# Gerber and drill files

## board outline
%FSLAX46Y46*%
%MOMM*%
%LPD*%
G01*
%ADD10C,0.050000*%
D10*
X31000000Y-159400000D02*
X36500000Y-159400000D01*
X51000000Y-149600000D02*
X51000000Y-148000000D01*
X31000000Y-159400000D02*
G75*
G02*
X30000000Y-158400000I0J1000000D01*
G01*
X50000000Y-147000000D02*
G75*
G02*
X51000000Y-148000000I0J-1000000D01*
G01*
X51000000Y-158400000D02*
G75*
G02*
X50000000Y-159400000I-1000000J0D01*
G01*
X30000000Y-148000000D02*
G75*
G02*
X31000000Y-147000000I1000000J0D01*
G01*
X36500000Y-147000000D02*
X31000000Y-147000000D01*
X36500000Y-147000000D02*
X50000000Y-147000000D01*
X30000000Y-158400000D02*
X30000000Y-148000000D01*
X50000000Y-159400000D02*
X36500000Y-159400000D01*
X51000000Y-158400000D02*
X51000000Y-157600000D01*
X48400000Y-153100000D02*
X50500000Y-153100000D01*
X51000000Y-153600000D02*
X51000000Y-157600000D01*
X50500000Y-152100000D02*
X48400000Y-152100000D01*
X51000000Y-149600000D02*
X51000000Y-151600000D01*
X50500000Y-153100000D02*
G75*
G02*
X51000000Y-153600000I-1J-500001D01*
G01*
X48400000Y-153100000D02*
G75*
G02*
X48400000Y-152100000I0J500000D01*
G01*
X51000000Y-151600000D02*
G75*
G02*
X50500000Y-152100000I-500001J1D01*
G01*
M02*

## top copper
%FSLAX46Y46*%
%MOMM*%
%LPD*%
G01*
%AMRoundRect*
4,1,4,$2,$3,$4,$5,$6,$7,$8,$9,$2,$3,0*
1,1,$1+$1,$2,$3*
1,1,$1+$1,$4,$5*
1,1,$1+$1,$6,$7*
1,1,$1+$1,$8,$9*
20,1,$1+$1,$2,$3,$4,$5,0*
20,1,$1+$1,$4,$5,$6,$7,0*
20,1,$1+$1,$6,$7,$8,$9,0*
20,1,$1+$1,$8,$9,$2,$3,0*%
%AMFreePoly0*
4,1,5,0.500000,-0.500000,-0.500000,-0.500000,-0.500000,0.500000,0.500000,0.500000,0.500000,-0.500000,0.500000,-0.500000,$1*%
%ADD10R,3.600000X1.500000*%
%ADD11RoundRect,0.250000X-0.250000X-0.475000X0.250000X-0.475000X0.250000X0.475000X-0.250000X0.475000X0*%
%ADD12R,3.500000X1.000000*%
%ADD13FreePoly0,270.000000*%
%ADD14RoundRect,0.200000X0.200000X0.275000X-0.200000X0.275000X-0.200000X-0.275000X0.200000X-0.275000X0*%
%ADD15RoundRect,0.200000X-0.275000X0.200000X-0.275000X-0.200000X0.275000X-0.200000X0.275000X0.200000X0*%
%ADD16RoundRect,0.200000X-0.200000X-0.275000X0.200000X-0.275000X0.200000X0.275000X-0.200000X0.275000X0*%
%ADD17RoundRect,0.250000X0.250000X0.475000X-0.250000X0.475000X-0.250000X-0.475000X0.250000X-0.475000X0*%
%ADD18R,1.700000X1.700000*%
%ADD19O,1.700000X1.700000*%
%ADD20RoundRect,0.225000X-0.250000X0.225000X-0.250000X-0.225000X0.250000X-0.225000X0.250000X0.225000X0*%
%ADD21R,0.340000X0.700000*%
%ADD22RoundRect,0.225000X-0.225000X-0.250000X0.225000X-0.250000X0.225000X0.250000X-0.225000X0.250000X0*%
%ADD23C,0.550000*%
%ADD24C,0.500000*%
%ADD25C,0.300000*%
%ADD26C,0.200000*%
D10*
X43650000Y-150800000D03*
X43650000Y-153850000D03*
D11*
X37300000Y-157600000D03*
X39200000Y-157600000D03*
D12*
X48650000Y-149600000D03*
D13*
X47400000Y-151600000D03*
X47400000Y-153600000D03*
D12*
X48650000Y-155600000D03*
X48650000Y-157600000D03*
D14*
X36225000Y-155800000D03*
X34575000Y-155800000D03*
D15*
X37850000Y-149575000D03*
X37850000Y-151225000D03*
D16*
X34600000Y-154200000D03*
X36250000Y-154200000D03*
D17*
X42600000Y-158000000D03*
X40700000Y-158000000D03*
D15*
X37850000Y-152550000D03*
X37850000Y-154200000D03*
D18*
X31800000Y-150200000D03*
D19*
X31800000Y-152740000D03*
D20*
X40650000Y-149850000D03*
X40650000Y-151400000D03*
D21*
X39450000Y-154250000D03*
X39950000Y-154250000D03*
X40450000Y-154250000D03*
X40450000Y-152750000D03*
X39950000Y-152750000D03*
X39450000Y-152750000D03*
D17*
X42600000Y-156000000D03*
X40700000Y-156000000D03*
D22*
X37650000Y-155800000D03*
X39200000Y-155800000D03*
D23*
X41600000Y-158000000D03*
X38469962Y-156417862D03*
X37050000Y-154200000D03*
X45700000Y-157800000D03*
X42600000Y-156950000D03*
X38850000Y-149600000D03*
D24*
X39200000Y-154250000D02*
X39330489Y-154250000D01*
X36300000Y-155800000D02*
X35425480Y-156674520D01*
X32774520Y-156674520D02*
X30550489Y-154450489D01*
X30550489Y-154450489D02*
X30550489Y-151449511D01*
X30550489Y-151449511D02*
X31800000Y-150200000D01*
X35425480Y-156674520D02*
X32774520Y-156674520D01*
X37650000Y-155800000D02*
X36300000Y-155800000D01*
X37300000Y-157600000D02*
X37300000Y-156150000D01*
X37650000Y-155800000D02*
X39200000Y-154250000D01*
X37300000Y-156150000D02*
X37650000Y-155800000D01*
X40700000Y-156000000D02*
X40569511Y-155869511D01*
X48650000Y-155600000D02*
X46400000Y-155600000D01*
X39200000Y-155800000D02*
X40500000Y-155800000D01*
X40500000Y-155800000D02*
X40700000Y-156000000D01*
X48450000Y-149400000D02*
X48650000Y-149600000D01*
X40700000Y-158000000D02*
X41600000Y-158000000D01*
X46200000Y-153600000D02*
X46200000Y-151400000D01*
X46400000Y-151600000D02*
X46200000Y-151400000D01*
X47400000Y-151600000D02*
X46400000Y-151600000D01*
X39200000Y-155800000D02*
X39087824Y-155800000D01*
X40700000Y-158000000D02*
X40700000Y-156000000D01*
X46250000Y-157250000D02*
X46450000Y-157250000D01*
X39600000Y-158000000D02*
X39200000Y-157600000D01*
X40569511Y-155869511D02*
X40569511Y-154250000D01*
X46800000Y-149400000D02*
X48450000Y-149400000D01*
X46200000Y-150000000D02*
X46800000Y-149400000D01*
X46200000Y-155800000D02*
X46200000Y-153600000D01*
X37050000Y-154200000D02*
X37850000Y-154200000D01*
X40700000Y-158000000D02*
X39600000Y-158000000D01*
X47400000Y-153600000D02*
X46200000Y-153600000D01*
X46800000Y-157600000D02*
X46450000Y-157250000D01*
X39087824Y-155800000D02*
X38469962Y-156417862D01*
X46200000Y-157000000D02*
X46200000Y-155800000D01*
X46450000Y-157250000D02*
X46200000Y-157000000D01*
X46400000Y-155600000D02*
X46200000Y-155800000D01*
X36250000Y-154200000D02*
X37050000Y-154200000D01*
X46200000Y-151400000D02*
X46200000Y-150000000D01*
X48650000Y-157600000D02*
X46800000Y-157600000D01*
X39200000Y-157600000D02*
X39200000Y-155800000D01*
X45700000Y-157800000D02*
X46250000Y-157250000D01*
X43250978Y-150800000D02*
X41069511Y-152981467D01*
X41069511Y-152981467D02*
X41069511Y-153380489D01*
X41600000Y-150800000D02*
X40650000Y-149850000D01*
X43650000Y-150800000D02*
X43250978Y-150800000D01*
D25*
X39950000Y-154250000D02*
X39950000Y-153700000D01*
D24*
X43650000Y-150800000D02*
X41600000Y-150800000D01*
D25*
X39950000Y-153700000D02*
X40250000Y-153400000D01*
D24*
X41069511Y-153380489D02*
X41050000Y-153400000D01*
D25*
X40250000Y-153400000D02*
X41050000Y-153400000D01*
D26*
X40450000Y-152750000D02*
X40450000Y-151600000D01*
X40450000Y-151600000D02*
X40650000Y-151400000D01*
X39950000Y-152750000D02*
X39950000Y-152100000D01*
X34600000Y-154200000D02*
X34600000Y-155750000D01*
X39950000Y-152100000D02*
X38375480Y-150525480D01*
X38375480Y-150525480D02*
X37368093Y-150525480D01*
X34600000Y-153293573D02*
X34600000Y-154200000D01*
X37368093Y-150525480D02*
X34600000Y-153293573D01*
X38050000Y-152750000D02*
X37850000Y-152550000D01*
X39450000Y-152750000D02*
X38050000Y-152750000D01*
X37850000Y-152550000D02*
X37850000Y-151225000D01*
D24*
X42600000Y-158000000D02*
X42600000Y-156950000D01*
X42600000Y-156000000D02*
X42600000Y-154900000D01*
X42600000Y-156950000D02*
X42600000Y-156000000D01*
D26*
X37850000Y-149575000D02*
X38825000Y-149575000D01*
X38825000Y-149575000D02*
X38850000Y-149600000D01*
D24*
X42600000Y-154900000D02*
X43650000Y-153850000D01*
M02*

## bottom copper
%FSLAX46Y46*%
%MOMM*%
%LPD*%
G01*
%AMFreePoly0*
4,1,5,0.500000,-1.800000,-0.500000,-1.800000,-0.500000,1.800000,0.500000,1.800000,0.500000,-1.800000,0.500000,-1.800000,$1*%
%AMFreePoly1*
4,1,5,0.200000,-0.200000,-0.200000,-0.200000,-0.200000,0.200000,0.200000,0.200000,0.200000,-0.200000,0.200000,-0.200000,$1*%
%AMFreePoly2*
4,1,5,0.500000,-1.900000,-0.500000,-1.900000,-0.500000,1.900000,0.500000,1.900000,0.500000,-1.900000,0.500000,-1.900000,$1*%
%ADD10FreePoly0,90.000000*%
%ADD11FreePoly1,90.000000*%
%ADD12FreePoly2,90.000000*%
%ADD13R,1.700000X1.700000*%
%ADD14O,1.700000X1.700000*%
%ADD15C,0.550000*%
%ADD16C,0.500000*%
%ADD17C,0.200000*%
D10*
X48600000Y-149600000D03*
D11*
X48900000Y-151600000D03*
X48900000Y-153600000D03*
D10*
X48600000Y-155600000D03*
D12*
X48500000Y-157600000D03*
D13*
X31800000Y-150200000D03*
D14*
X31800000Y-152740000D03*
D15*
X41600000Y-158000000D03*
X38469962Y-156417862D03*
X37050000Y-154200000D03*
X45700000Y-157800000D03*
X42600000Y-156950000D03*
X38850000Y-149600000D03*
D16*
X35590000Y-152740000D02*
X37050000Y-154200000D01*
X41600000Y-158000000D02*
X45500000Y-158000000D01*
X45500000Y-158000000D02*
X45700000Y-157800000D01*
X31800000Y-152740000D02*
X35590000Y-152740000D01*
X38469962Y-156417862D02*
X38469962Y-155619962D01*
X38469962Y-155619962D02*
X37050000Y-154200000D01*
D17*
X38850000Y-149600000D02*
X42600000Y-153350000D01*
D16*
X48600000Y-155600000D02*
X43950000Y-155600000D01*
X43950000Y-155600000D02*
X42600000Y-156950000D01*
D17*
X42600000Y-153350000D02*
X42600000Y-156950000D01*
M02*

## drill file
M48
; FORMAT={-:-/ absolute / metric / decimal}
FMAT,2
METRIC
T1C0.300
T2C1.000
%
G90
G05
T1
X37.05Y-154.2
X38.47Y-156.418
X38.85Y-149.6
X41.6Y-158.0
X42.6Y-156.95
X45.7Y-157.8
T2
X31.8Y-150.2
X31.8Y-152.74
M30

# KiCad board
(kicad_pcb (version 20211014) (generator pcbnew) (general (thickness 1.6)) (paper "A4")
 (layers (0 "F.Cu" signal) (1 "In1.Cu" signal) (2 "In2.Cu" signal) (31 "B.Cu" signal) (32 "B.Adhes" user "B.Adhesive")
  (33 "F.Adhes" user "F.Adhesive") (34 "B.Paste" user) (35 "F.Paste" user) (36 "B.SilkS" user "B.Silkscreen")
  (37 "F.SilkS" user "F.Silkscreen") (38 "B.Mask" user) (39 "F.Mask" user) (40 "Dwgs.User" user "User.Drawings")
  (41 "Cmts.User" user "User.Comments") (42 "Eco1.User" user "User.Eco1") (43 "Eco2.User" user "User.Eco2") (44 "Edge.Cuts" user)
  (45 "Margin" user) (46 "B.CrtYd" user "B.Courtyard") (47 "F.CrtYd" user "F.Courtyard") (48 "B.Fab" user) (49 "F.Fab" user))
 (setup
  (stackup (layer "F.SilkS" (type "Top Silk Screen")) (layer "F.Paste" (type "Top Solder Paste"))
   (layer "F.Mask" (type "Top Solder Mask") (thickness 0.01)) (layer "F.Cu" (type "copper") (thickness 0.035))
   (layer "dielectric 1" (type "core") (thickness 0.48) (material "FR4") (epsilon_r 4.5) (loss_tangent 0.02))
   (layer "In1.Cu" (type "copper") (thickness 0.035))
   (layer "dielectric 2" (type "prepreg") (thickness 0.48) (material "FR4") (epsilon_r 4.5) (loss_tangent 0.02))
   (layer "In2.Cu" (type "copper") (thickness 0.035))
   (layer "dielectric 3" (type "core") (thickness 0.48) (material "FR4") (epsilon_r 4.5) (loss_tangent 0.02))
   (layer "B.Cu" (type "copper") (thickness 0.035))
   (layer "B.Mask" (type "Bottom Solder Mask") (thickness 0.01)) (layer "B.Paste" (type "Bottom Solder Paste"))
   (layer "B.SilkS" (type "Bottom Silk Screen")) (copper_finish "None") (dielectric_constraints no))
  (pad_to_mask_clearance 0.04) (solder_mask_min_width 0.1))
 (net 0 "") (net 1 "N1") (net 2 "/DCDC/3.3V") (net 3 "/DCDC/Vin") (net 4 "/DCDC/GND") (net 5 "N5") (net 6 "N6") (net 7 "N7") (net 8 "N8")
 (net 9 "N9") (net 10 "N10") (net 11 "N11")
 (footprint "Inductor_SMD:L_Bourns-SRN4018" (layer "F.Cu") (at 43.65 152.325 -90)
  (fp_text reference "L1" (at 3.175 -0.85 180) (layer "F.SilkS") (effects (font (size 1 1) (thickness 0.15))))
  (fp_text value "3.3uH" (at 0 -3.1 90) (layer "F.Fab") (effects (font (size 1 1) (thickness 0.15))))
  (pad "1" smd rect locked (at -1.525 0 270) (size 1.5 3.6) (layers "F.Cu" "F.Paste" "F.Mask") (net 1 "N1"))
  (pad "2" smd rect locked (at 1.525 0 270) (size 1.5 3.6) (layers "F.Cu" "F.Paste" "F.Mask") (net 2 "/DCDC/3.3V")))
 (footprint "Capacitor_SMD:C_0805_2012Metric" (layer "F.Cu") (at 38.25 157.6)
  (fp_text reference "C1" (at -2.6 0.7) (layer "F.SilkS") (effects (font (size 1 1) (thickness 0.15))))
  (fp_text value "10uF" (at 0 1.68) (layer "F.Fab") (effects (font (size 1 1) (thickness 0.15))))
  (pad "1" smd roundrect locked (at -0.95 0) (size 1 1.45) (layers "F.Cu" "F.Paste" "F.Mask") (roundrect_rratio 0.25) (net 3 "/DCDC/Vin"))
  (pad "2" smd roundrect locked (at 0.95 0) (size 1 1.45) (layers "F.Cu" "F.Paste" "F.Mask") (roundrect_rratio 0.25) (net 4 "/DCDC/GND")))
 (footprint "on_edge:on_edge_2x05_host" (layer "F.Cu") (at 51 153.6 -90)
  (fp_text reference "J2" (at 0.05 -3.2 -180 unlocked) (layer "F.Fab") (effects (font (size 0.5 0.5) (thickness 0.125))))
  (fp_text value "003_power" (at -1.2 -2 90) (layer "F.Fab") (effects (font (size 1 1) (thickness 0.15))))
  (fp_line (start -0.5 2.6) (end -0.5 0.5) (layer "Edge.Cuts") (width 0.05))
  (fp_line (start 0 0) (end 4 0) (layer "Edge.Cuts") (width 0.05))
  (fp_line (start -1.5 0.5) (end -1.5 2.6) (layer "Edge.Cuts") (width 0.05))
  (fp_line (start -4 0) (end -2 0) (layer "Edge.Cuts") (width 0.05))
  (fp_arc (start -0.5 0.5) (mid -0.353553 0.146447) (end 0 0) (layer "Edge.Cuts") (width 0.05))
  (fp_arc (start -0.5 2.6) (mid -1 3.1) (end -1.5 2.6) (layer "Edge.Cuts") (width 0.05))
  (fp_arc (start -2 0) (mid -1.646447 0.146447) (end -1.5 0.5) (layer "Edge.Cuts") (width 0.05))
  (pad "1" smd rect locked (at -4 2.35 270) (size 1 3.5) (layers "F.Cu" "F.Mask") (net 4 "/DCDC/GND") (zone_connect 0))
  (pad "2" smd custom locked (at -2 3.6 270) (size 1 1) (layers "F.Cu" "F.Mask") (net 4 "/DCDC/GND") (zone_connect 0)
   (options (clearance outline) (anchor rect)) (primitives))
  (pad "3" smd custom locked (at 0 3.6 270) (size 1 1) (layers "F.Cu" "F.Mask") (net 4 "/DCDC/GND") (zone_connect 0)
   (options (clearance outline) (anchor rect)) (primitives))
  (pad "4" smd rect locked (at 2 2.35 270) (size 1 3.5) (layers "F.Cu" "F.Mask") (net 4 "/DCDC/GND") (zone_connect 0))
  (pad "5" smd rect locked (at 4 2.35 270) (size 1 3.5) (layers "F.Cu" "F.Mask") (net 4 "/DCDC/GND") (zone_connect 0))
  (pad "6" smd custom locked (at -4 2.4 90) (size 1 3.6) (layers "B.Cu" "B.Mask") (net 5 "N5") (zone_connect 0)
   (options (clearance outline) (anchor rect)) (primitives))
  (pad "7" smd custom locked (at -2 2.1 90) (size 0.4 0.4) (layers "B.Cu" "B.Mask") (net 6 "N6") (zone_connect 0)
   (options (clearance outline) (anchor rect)) (primitives))
  (pad "8" smd custom locked (at 0 2.1 90) (size 0.4 0.4) (layers "B.Cu" "B.Mask") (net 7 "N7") (zone_connect 0)
   (options (clearance outline) (anchor rect)) (primitives))
  (pad "9" smd custom locked (at 2 2.4 90) (size 1 3.6) (layers "B.Cu" "B.Mask") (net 2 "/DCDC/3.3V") (zone_connect 0)
   (options (clearance outline) (anchor rect)) (primitives))
  (pad "10" smd custom locked (at 4 2.5 90) (size 1 3.8) (layers "B.Cu" "B.Mask") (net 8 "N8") (zone_connect 0)
   (options (clearance outline) (anchor rect)) (primitives)))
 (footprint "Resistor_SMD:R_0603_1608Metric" (layer "F.Cu") (at 35.4 155.8 180)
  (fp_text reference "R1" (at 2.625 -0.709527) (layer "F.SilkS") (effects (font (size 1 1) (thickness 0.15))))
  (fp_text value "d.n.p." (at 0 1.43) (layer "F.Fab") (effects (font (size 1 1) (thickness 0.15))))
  (pad "1" smd roundrect locked (at -0.825 0 180) (size 0.8 0.95) (layers "F.Cu" "F.Paste" "F.Mask") (roundrect_rratio 0.25)
   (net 3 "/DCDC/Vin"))
  (pad "2" smd roundrect locked (at 0.825 0 180) (size 0.8 0.95) (layers "F.Cu" "F.Paste" "F.Mask") (roundrect_rratio 0.25) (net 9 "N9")))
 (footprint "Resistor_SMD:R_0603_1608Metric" (layer "F.Cu") (at 37.85 150.4 -90)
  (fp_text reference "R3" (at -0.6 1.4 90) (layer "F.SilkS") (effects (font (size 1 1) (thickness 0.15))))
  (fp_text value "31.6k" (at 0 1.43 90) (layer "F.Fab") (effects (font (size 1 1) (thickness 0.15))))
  (pad "1" smd roundrect locked (at -0.825 0 270) (size 0.8 0.95) (layers "F.Cu" "F.Paste" "F.Mask") (roundrect_rratio 0.25)
   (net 2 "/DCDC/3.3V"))
  (pad "2" smd roundrect locked (at 0.825 0 270) (size 0.8 0.95) (layers "F.Cu" "F.Paste" "F.Mask") (roundrect_rratio 0.25) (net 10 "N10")))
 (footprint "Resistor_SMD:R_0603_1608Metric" (layer "F.Cu") (at 35.425 154.2)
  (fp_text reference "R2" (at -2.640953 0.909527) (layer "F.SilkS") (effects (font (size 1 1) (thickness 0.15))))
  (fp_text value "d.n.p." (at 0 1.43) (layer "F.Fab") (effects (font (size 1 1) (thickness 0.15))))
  (pad "1" smd roundrect locked (at -0.825 0) (size 0.8 0.95) (layers "F.Cu" "F.Paste" "F.Mask") (roundrect_rratio 0.25) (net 9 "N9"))
  (pad "2" smd roundrect locked (at 0.825 0) (size 0.8 0.95) (layers "F.Cu" "F.Paste" "F.Mask") (roundrect_rratio 0.25) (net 4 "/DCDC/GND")))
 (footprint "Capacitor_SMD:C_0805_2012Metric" (layer "F.Cu") (at 41.65 158 180)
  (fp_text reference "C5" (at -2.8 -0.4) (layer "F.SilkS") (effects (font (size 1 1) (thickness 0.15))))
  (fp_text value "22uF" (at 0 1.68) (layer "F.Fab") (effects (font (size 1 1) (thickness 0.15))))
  (pad "1" smd roundrect locked (at -0.95 0 180) (size 1 1.45) (layers "F.Cu" "F.Paste" "F.Mask") (roundrect_rratio 0.25)
   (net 2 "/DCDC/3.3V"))
  (pad "2" smd roundrect locked (at 0.95 0 180) (size 1 1.45) (layers "F.Cu" "F.Paste" "F.Mask") (roundrect_rratio 0.25) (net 4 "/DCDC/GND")))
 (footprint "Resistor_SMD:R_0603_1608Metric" (layer "F.Cu") (at 37.85 153.375 -90)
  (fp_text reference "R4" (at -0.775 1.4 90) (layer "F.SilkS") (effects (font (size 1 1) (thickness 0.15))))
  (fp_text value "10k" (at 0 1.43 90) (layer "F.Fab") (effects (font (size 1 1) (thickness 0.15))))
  (pad "1" smd roundrect locked (at -0.825 0 270) (size 0.8 0.95) (layers "F.Cu" "F.Paste" "F.Mask") (roundrect_rratio 0.25) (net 10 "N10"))
  (pad "2" smd roundrect locked (at 0.825 0 270) (size 0.8 0.95) (layers "F.Cu" "F.Paste" "F.Mask") (roundrect_rratio 0.25)
   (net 4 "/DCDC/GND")))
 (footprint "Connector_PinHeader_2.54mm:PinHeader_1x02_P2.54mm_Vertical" (layer "F.Cu") (at 31.8 150.2)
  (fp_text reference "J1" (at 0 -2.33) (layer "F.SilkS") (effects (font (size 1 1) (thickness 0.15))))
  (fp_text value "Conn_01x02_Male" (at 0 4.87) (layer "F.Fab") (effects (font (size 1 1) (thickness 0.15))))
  (pad "1" thru_hole rect locked (at 0 0) (size 1.7 1.7) (drill 1) (layers *.Cu *.Mask) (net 3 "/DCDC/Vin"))
  (pad "2" thru_hole oval locked (at 0 2.54) (size 1.7 1.7) (drill 1) (layers *.Cu *.Mask) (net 4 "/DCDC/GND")))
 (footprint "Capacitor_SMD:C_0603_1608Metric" (layer "F.Cu") (at 40.65 150.625 -90)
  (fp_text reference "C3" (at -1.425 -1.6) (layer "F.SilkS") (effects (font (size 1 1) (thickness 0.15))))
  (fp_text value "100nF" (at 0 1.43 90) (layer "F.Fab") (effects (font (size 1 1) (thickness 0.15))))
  (pad "1" smd roundrect locked (at -0.775 0 270) (size 0.9 0.95) (layers "F.Cu" "F.Paste" "F.Mask") (roundrect_rratio 0.25) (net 1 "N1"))
  (pad "2" smd roundrect locked (at 0.775 0 270) (size 0.9 0.95) (layers "F.Cu" "F.Paste" "F.Mask") (roundrect_rratio 0.25) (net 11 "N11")))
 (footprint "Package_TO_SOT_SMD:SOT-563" (layer "F.Cu") (at 39.95 153.5 90)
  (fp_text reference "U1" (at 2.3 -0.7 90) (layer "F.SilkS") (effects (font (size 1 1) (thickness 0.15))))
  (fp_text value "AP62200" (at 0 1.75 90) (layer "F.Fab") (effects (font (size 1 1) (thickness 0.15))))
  (pad "1" smd rect locked (at -0.75 -0.5 90) (size 0.7 0.34) (layers "F.Cu" "F.Paste" "F.Mask") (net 3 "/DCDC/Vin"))
  (pad "2" smd rect locked (at -0.75 0 90) (size 0.7 0.34) (layers "F.Cu" "F.Paste" "F.Mask") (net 1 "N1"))
  (pad "3" smd rect locked (at -0.75 0.5 90) (size 0.7 0.34) (layers "F.Cu" "F.Paste" "F.Mask") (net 4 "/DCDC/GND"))
  (pad "4" smd rect locked (at 0.75 0.5 90) (size 0.7 0.34) (layers "F.Cu" "F.Paste" "F.Mask") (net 11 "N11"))
  (pad "5" smd rect locked (at 0.75 0 90) (size 0.7 0.34) (layers "F.Cu" "F.Paste" "F.Mask") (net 9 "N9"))
  (pad "6" smd rect locked (at 0.75 -0.5 90) (size 0.7 0.34) (layers "F.Cu" "F.Paste" "F.Mask") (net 10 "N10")))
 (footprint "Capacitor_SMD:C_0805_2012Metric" (layer "F.Cu") (at 41.65 156 180)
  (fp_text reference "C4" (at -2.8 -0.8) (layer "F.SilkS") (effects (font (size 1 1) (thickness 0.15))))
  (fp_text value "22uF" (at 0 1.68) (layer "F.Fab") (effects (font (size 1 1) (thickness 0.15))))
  (pad "1" smd roundrect locked (at -0.95 0 180) (size 1 1.45) (layers "F.Cu" "F.Paste" "F.Mask") (roundrect_rratio 0.25)
   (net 2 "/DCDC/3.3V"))
  (pad "2" smd roundrect locked (at 0.95 0 180) (size 1 1.45) (layers "F.Cu" "F.Paste" "F.Mask") (roundrect_rratio 0.25) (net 4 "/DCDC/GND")))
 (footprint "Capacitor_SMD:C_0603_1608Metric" (layer "F.Cu") (at 38.425 155.8)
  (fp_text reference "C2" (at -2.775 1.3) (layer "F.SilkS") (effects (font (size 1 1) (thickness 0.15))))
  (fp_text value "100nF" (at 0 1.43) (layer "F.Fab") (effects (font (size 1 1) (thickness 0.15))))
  (pad "1" smd roundrect locked (at -0.775 0) (size 0.9 0.95) (layers "F.Cu" "F.Paste" "F.Mask") (roundrect_rratio 0.25) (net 3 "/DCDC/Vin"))
  (pad "2" smd roundrect locked (at 0.775 0) (size 0.9 0.95) (layers "F.Cu" "F.Paste" "F.Mask") (roundrect_rratio 0.25) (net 4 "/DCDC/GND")))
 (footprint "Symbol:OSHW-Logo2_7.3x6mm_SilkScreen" (layer "B.Cu") (at 39.984047 156.209527 180)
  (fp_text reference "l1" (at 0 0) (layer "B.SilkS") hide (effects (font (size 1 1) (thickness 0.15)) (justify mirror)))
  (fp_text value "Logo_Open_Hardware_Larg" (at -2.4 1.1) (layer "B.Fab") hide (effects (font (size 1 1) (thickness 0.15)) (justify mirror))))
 (gr_line (start 31 159.4) (end 36.5 159.4) (layer "Edge.Cuts") (width 0.05))
 (gr_line (start 51 149.6) (end 51 148) (layer "Edge.Cuts") (width 0.05))
 (gr_arc (start 31 159.4) (mid 30.292893 159.107107) (end 30 158.4) (layer "Edge.Cuts") (width 0.05))
 (gr_arc (start 50 147) (mid 50.707107 147.292893) (end 51 148) (layer "Edge.Cuts") (width 0.05))
 (gr_arc (start 51 158.4) (mid 50.707107 159.107107) (end 50 159.4) (layer "Edge.Cuts") (width 0.05))
 (gr_arc (start 30 148) (mid 30.292893 147.292893) (end 31 147) (layer "Edge.Cuts") (width 0.05))
 (gr_line (start 36.5 147) (end 31 147) (layer "Edge.Cuts") (width 0.05))
 (gr_line (start 36.5 147) (end 50 147) (layer "Edge.Cuts") (width 0.05))
 (gr_line (start 30 158.4) (end 30 148) (layer "Edge.Cuts") (width 0.05))
 (gr_line (start 50 159.4) (end 36.5 159.4) (layer "Edge.Cuts") (width 0.05))
 (gr_line (start 51 158.4) (end 51 157.6) (layer "Edge.Cuts") (width 0.05))
 (segment (start 39.2 154.25) (end 39.330489 154.25) (width 0.5) (layer "F.Cu") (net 3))
 (segment (start 36.3 155.8) (end 35.42548 156.67452) (width 0.5) (layer "F.Cu") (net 3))
 (segment (start 32.77452 156.67452) (end 30.550489 154.450489) (width 0.5) (layer "F.Cu") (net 3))
 (segment (start 30.550489 154.450489) (end 30.550489 151.449511) (width 0.5) (layer "F.Cu") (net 3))
 (segment (start 30.550489 151.449511) (end 31.8 150.2) (width 0.5) (layer "F.Cu") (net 3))
 (segment (start 35.42548 156.67452) (end 32.77452 156.67452) (width 0.5) (layer "F.Cu") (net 3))
 (segment (start 37.65 155.8) (end 36.3 155.8) (width 0.5) (layer "F.Cu") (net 3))
 (segment (start 37.3 157.6) (end 37.3 156.15) (width 0.5) (layer "F.Cu") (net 3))
 (segment (start 37.65 155.8) (end 39.2 154.25) (width 0.5) (layer "F.Cu") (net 3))
 (segment (start 37.3 156.15) (end 37.65 155.8) (width 0.5) (layer "F.Cu") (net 3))
 (segment (start 40.7 156) (end 40.569511 155.869511) (width 0.5) (layer "F.Cu") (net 4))
 (segment (start 48.65 155.6) (end 46.4 155.6) (width 0.5) (layer "F.Cu") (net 4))
 (segment (start 39.2 155.8) (end 40.5 155.8) (width 0.5) (layer "F.Cu") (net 4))
 (segment (start 40.5 155.8) (end 40.7 156) (width 0.5) (layer "F.Cu") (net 4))
 (segment (start 48.45 149.4) (end 48.65 149.6) (width 0.5) (layer "F.Cu") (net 4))
 (segment (start 40.7 158) (end 41.6 158) (width 0.5) (layer "F.Cu") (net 4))
 (segment (start 46.2 153.6) (end 46.2 151.4) (width 0.5) (layer "F.Cu") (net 4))
 (segment (start 46.4 151.6) (end 46.2 151.4) (width 0.5) (layer "F.Cu") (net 4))
 (segment (start 47.4 151.6) (end 46.4 151.6) (width 0.5) (layer "F.Cu") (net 4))
 (segment (start 39.2 155.8) (end 39.087824 155.8) (width 0.5) (layer "F.Cu") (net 4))
 (segment (start 40.7 158) (end 40.7 156) (width 0.5) (layer "F.Cu") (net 4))
 (segment (start 46.25 157.25) (end 46.45 157.25) (width 0.5) (layer "F.Cu") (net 4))
 (segment (start 39.6 158) (end 39.2 157.6) (width 0.5) (layer "F.Cu") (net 4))
 (segment (start 40.569511 155.869511) (end 40.569511 154.25) (width 0.5) (layer "F.Cu") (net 4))
 (segment (start 46.8 149.4) (end 48.45 149.4) (width 0.5) (layer "F.Cu") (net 4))
 (segment (start 46.2 150) (end 46.8 149.4) (width 0.5) (layer "F.Cu") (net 4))
 (segment (start 46.2 155.8) (end 46.2 153.6) (width 0.5) (layer "F.Cu") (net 4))
 (segment (start 37.05 154.2) (end 37.85 154.2) (width 0.5) (layer "F.Cu") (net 4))
 (segment (start 40.7 158) (end 39.6 158) (width 0.5) (layer "F.Cu") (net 4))
 (segment (start 47.4 153.6) (end 46.2 153.6) (width 0.5) (layer "F.Cu") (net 4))
 (segment (start 46.8 157.6) (end 46.45 157.25) (width 0.5) (layer "F.Cu") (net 4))
 (segment (start 39.087824 155.8) (end 38.469962 156.417862) (width 0.5) (layer "F.Cu") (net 4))
 (segment (start 46.2 157) (end 46.2 155.8) (width 0.5) (layer "F.Cu") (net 4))
 (segment (start 46.45 157.25) (end 46.2 157) (width 0.5) (layer "F.Cu") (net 4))
 (segment (start 46.4 155.6) (end 46.2 155.8) (width 0.5) (layer "F.Cu") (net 4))
 (segment (start 36.25 154.2) (end 37.05 154.2) (width 0.5) (layer "F.Cu") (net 4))
 (segment (start 46.2 151.4) (end 46.2 150) (width 0.5) (layer "F.Cu") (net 4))
 (segment (start 48.65 157.6) (end 46.8 157.6) (width 0.5) (layer "F.Cu") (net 4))
 (segment (start 39.2 157.6) (end 39.2 155.8) (width 0.5) (layer "F.Cu") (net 4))
 (segment (start 45.7 157.8) (end 46.25 157.25) (width 0.5) (layer "F.Cu") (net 4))
 (via (at 41.6 158) (size 0.55) (drill 0.3) (layers "F.Cu" "B.Cu") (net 4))
 (via (at 38.469962 156.417862) (size 0.55) (drill 0.3) (layers "F.Cu" "B.Cu") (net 4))
 (via (at 37.05 154.2) (size 0.55) (drill 0.3) (layers "F.Cu" "B.Cu") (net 4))
 (via (at 45.7 157.8) (size 0.55) (drill 0.3) (layers "F.Cu" "B.Cu") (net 4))
 (segment (start 35.59 152.74) (end 37.05 154.2) (width 0.5) (layer "B.Cu") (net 4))
 (segment (start 41.6 158) (end 45.5 158) (width 0.5) (layer "B.Cu") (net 4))
 (segment (start 45.5 158) (end 45.7 157.8) (width 0.5) (layer "B.Cu") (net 4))
 (segment (start 31.8 152.74) (end 35.59 152.74) (width 0.5) (layer "B.Cu") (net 4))
 (segment (start 38.469962 156.417862) (end 38.469962 155.619962) (width 0.5) (layer "B.Cu") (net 4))
 (segment (start 38.469962 155.619962) (end 37.05 154.2) (width 0.5) (layer "B.Cu") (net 4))
 (segment (start 43.250978 150.8) (end 41.069511 152.981467) (width 0.5) (layer "F.Cu") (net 1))
 (segment (start 41.069511 152.981467) (end 41.069511 153.380489) (width 0.5) (layer "F.Cu") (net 1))
 (segment (start 41.6 150.8) (end 40.65 149.85) (width 0.5) (layer "F.Cu") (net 1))
 (segment (start 43.65 150.8) (end 43.250978 150.8) (width 0.5) (layer "F.Cu") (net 1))
 (segment (start 39.95 154.25) (end 39.95 153.7) (width 0.3) (layer "F.Cu") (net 1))
 (segment (start 43.65 150.8) (end 41.6 150.8) (width 0.5) (layer "F.Cu") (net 1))
 (segment (start 39.95 153.7) (end 40.25 153.4) (width 0.3) (layer "F.Cu") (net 1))
 (segment (start 41.069511 153.380489) (end 41.05 153.4) (width 0.5) (layer "F.Cu") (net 1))
 (segment (start 40.25 153.4) (end 41.05 153.4) (width 0.3) (layer "F.Cu") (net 1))
 (segment (start 40.45 152.75) (end 40.45 151.6) (width 0.2) (layer "F.Cu") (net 11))
 (segment (start 40.45 151.6) (end 40.65 151.4) (width 0.2) (layer "F.Cu") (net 11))
 (segment (start 39.95 152.75) (end 39.95 152.1) (width 0.2) (layer "F.Cu") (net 9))
 (segment (start 34.6 154.2) (end 34.6 155.75) (width 0.2) (layer "F.Cu") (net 9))
 (segment (start 39.95 152.1) (end 38.37548 150.52548) (width 0.2) (layer "F.Cu") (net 9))
 (segment (start 38.37548 150.52548) (end 37.368093 150.52548) (width 0.2) (layer "F.Cu") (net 9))
 (segment (start 34.6 153.293573) (end 34.6 154.2) (width 0.2) (layer "F.Cu") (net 9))
 (segment (start 37.368093 150.52548) (end 34.6 153.293573) (width 0.2) (layer "F.Cu") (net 9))
 (segment (start 38.05 152.75) (end 37.85 152.55) (width 0.2) (layer "F.Cu") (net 10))
 (segment (start 39.45 152.75) (end 38.05 152.75) (width 0.2) (layer "F.Cu") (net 10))
 (segment (start 37.85 152.55) (end 37.85 151.225) (width 0.2) (layer "F.Cu") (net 10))
 (segment (start 42.6 158) (end 42.6 156.95) (width 0.5) (layer "F.Cu") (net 2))
 (segment (start 42.6 156) (end 42.6 154.9) (width 0.5) (layer "F.Cu") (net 2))
 (segment (start 42.6 156.95) (end 42.6 156) (width 0.5) (layer "F.Cu") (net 2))
 (segment (start 37.85 149.575) (end 38.825 149.575) (width 0.2) (layer "F.Cu") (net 2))
 (segment (start 38.825 149.575) (end 38.85 149.6) (width 0.2) (layer "F.Cu") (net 2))
 (segment (start 42.6 154.9) (end 43.65 153.85) (width 0.5) (layer "F.Cu") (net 2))
 (via (at 42.6 156.95) (size 0.55) (drill 0.3) (layers "F.Cu" "B.Cu") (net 2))
 (via (at 38.85 149.6) (size 0.55) (drill 0.3) (layers "F.Cu" "B.Cu") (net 2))
 (segment (start 38.85 149.6) (end 42.6 153.35) (width 0.2) (layer "B.Cu") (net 2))
 (segment (start 48.6 155.6) (end 43.95 155.6) (width 0.5) (layer "B.Cu") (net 2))
 (segment (start 43.95 155.6) (end 42.6 156.95) (width 0.5) (layer "B.Cu") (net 2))
 (segment (start 42.6 153.35) (end 42.6 156.95) (width 0.2) (layer "B.Cu") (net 2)))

